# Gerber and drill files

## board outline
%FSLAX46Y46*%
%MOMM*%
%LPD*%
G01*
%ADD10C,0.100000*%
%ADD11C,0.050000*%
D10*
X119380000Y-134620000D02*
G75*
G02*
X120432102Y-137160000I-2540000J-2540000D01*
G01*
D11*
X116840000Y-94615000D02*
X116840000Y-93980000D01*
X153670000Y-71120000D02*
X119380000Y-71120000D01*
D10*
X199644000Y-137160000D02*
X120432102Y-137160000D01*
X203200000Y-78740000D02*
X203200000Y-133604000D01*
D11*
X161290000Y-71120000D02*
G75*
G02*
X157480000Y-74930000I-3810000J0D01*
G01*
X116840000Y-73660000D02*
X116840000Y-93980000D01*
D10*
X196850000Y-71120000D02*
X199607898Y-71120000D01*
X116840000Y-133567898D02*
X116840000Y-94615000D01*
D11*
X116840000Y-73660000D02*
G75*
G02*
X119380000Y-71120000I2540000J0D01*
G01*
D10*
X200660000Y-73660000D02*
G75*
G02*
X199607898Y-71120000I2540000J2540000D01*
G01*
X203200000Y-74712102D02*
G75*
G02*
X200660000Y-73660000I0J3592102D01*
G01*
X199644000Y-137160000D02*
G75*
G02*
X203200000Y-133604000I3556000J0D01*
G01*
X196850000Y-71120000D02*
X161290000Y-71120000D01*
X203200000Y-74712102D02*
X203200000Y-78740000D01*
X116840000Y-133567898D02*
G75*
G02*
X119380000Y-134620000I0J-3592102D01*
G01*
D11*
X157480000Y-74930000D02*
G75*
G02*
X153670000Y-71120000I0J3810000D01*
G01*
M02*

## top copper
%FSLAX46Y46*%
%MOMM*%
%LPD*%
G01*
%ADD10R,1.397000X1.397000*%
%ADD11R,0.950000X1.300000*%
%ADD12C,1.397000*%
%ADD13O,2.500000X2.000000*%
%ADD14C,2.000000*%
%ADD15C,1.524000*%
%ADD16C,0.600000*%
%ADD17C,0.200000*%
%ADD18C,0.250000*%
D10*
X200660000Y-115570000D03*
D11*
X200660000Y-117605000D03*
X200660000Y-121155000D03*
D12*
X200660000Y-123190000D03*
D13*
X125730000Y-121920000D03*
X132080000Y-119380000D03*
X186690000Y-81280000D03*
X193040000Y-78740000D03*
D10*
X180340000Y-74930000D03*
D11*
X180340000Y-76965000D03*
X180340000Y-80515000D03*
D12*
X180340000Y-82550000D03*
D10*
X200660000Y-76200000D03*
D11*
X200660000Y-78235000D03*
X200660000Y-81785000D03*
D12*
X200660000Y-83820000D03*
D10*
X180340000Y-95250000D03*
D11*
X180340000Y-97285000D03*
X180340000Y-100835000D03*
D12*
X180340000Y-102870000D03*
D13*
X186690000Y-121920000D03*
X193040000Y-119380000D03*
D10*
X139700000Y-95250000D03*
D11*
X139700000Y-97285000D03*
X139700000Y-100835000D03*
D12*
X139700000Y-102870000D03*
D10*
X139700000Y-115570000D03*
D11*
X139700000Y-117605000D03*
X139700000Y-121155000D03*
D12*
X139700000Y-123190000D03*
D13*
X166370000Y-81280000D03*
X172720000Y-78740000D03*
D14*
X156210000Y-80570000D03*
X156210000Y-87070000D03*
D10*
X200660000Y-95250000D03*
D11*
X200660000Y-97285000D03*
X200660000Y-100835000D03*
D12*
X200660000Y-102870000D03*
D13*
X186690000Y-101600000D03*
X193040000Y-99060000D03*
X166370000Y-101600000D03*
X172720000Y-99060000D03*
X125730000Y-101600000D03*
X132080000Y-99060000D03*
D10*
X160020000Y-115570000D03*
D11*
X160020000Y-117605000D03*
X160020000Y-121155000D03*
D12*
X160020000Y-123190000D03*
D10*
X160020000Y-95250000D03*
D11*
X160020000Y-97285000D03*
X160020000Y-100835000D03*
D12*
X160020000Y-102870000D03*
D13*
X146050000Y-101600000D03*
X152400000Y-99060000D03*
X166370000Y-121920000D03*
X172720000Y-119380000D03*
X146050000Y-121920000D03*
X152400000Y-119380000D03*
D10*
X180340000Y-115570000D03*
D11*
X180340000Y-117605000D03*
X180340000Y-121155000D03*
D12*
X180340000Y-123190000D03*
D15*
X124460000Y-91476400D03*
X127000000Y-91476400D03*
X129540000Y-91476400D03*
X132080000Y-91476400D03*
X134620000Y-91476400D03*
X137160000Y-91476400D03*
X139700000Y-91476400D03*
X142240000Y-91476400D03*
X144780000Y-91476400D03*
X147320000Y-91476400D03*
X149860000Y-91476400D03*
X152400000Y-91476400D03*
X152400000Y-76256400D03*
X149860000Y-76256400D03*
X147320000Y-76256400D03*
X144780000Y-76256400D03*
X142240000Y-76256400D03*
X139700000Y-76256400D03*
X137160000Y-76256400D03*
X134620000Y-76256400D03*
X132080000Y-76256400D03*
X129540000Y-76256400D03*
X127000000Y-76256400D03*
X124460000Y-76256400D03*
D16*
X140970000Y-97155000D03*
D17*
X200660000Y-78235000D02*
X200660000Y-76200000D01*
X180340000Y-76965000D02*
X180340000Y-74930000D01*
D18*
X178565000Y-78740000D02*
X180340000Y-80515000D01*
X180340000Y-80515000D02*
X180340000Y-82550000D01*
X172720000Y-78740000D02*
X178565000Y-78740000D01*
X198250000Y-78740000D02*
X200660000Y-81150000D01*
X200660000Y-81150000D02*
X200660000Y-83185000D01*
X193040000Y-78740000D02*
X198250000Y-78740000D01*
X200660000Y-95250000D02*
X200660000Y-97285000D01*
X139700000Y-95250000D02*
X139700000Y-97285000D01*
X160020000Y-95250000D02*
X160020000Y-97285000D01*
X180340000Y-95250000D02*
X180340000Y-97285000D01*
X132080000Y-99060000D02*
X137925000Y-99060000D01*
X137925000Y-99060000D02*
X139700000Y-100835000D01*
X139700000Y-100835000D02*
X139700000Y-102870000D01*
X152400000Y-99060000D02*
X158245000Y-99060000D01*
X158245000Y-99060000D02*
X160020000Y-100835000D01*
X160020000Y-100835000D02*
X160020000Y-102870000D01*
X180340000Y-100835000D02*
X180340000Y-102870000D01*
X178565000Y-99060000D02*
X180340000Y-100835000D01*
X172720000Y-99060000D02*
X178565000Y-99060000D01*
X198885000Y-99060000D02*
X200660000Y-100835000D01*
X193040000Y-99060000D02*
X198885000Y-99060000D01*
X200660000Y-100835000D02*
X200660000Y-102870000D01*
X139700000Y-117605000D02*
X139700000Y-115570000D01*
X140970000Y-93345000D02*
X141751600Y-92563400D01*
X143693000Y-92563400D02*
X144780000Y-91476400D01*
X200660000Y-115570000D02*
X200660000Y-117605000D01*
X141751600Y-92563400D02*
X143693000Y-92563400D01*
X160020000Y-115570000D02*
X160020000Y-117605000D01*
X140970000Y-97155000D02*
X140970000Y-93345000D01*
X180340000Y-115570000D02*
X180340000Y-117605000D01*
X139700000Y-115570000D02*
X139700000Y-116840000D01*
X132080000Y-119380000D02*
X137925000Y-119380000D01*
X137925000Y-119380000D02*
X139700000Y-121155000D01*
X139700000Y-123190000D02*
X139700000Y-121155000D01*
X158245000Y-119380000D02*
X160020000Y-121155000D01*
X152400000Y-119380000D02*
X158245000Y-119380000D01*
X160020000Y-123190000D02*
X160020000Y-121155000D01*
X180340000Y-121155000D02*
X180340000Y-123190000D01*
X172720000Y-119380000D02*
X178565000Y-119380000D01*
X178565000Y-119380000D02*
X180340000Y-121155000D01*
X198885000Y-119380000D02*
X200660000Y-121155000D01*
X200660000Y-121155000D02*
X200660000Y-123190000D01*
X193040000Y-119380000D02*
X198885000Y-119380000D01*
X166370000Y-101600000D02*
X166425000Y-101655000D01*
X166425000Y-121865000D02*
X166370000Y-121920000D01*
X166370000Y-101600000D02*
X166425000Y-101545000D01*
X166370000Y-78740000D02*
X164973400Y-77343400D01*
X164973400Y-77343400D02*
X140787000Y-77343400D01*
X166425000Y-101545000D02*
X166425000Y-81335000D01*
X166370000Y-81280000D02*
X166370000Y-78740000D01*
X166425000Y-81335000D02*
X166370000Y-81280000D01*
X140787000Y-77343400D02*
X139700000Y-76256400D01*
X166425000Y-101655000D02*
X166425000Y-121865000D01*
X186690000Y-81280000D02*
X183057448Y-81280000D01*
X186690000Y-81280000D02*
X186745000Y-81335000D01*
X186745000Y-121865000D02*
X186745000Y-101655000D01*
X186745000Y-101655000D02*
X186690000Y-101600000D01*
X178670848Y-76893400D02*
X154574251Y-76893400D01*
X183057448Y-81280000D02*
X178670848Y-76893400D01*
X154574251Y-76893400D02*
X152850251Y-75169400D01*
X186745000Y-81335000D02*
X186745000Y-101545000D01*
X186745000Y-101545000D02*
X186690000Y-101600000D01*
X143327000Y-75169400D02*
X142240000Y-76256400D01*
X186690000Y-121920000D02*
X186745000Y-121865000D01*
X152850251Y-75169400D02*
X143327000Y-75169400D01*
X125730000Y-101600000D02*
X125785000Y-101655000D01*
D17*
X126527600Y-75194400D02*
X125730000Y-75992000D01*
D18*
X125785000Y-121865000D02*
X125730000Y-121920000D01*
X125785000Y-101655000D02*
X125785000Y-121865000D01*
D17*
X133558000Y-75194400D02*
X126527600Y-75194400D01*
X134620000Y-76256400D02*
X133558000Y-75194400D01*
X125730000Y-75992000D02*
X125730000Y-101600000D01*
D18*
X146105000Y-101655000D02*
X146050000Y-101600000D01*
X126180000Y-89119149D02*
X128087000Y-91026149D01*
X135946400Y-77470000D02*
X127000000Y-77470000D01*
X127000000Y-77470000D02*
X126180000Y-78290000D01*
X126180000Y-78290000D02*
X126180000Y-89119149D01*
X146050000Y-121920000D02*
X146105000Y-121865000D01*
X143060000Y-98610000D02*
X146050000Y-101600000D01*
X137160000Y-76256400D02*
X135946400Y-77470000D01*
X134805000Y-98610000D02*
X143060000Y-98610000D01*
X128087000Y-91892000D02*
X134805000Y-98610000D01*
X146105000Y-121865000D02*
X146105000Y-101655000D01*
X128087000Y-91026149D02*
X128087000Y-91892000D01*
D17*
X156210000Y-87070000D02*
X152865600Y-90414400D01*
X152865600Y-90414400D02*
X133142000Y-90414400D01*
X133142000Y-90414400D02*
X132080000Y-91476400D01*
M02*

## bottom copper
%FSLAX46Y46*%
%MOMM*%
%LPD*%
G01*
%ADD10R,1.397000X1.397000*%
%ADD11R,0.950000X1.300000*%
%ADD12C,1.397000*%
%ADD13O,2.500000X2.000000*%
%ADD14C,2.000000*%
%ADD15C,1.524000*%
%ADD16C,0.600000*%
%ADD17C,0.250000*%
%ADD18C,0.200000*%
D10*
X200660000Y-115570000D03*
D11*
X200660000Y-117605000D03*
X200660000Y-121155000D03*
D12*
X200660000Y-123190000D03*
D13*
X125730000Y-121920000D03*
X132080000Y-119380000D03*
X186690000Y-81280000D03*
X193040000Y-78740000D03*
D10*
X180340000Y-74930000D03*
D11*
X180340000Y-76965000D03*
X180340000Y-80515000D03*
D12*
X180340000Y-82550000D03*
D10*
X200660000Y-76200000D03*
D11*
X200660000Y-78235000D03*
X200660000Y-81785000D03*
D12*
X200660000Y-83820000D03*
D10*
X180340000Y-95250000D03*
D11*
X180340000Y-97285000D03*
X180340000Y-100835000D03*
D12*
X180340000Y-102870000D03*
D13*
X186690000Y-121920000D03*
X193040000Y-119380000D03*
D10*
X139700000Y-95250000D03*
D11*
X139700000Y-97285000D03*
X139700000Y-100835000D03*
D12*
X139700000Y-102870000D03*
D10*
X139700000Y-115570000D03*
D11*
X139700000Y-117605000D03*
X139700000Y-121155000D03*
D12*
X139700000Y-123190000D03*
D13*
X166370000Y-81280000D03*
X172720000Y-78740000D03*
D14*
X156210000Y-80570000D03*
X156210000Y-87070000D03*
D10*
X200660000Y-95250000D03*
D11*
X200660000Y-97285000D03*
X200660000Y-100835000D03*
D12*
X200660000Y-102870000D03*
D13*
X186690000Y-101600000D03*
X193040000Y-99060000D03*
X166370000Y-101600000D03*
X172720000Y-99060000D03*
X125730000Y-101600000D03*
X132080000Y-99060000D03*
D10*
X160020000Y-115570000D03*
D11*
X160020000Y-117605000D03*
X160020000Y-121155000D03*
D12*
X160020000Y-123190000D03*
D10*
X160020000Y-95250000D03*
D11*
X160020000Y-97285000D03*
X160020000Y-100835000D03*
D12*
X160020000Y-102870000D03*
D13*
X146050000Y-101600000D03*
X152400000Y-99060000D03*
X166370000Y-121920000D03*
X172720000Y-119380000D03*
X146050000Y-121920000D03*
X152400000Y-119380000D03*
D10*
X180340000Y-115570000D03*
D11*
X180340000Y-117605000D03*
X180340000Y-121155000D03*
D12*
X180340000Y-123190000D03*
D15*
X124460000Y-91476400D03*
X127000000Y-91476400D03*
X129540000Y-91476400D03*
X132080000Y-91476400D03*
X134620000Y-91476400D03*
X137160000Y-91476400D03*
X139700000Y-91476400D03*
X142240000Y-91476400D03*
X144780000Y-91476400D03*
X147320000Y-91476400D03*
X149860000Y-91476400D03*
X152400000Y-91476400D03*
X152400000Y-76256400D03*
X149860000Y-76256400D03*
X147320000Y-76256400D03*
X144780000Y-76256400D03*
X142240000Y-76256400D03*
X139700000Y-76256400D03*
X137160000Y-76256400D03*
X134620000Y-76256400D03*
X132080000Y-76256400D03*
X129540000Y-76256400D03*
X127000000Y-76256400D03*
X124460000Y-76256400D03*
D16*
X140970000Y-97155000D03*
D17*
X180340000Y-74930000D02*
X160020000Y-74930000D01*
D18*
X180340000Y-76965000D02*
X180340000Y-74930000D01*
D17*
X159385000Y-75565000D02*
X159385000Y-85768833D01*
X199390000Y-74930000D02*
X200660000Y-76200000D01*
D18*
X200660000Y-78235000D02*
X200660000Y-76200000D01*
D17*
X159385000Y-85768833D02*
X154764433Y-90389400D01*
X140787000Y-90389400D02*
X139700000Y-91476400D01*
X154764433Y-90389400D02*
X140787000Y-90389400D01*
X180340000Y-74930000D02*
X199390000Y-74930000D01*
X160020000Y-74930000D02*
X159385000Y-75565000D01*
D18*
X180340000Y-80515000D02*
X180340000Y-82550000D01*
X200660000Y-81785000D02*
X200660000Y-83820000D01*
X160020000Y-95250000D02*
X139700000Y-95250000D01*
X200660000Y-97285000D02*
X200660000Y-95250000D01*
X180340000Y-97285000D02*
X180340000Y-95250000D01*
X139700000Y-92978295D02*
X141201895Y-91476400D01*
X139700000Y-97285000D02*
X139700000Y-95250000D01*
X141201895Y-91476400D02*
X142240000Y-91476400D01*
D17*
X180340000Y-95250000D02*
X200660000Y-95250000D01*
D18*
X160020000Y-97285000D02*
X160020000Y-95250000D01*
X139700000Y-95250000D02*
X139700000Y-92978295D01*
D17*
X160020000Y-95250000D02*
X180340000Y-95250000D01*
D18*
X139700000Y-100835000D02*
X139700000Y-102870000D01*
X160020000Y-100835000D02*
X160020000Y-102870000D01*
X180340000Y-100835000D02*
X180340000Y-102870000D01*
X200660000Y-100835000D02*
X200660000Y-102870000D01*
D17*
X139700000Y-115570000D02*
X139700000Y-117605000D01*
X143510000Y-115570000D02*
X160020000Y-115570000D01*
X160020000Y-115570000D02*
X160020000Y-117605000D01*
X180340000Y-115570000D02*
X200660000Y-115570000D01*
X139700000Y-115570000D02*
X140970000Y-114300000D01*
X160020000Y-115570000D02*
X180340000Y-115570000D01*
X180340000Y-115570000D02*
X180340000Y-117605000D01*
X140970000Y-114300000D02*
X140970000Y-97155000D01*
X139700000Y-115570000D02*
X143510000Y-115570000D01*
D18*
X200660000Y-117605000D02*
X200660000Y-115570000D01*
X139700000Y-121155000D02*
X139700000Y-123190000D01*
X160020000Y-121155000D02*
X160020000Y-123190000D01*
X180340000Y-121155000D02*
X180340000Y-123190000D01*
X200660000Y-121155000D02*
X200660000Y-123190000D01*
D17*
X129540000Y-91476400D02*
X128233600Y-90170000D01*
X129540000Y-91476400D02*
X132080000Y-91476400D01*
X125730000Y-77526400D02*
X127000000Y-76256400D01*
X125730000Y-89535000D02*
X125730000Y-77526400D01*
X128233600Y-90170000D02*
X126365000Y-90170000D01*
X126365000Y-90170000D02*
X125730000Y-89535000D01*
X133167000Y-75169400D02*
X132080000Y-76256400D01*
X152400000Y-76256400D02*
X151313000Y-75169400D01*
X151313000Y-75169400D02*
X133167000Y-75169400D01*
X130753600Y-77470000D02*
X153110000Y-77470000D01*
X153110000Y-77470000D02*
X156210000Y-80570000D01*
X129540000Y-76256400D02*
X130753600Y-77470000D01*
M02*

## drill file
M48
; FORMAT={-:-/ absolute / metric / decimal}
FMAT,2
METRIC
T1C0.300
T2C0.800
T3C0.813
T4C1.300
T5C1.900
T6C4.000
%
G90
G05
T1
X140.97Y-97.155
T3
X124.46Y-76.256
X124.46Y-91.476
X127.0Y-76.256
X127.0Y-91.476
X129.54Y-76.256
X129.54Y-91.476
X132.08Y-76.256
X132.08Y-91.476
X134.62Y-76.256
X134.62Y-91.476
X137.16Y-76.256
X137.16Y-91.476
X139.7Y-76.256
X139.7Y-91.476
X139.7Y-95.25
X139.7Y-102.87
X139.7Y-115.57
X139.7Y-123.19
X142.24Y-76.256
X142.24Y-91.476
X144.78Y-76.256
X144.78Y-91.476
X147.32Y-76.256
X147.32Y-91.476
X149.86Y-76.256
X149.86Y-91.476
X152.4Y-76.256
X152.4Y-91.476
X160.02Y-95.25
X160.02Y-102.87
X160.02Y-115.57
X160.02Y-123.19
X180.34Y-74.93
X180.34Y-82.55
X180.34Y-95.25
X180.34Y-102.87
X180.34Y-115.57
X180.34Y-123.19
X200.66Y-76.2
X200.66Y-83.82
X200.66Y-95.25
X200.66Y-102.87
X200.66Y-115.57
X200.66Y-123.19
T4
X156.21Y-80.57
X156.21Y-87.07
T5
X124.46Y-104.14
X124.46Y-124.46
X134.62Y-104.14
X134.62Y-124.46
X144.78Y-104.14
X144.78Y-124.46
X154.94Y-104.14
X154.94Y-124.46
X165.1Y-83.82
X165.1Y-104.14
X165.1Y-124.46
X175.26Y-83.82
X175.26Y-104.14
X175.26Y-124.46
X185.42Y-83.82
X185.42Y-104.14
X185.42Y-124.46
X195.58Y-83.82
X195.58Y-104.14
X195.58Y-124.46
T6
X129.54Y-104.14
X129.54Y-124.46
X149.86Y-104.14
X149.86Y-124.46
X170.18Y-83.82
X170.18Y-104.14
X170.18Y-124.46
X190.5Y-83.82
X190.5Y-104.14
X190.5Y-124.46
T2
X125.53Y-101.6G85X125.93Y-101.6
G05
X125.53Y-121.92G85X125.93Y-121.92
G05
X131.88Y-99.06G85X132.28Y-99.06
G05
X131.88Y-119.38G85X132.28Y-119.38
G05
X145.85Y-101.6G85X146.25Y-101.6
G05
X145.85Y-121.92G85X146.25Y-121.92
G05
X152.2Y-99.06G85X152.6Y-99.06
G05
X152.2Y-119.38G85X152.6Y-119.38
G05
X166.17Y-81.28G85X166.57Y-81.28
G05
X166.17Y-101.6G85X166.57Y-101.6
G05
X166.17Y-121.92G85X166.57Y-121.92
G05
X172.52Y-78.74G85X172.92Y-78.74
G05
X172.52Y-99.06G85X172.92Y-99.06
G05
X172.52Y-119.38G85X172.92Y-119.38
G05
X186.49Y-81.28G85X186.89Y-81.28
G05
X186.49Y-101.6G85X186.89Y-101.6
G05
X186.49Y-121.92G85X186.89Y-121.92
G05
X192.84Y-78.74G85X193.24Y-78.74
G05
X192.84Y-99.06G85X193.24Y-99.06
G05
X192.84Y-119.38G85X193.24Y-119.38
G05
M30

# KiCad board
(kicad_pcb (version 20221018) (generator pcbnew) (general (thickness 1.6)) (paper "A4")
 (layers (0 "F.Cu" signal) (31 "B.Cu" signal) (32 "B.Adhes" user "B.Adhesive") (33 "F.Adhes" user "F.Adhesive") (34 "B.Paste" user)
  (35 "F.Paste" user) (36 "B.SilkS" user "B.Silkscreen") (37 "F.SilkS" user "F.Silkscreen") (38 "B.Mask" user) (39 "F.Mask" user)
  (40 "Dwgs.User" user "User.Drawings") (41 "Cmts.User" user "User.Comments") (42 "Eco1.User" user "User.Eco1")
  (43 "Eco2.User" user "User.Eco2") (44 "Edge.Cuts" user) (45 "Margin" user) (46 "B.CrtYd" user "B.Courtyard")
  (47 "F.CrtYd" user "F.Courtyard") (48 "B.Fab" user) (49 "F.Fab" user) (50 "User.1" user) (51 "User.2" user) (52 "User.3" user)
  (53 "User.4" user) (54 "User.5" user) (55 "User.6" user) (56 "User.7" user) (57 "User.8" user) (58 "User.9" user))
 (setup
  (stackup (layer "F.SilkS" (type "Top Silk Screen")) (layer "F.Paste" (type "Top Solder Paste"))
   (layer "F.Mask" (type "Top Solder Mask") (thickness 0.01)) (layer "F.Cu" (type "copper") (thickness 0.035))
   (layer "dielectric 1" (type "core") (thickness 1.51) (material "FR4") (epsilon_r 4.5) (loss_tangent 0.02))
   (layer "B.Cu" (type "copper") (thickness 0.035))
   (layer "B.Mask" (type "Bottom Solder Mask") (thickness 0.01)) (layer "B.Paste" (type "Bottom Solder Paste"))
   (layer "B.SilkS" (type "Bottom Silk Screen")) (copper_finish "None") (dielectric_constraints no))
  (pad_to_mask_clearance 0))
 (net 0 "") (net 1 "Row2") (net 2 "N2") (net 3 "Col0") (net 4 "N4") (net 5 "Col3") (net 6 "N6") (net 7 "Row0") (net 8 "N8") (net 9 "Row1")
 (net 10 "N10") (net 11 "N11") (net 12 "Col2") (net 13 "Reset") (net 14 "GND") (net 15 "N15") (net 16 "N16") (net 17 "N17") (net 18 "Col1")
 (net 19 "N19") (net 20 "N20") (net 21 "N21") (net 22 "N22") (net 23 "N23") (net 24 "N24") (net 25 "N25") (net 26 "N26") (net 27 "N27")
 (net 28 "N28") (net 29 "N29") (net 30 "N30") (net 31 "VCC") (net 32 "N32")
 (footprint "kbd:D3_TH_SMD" (layer "F.Cu") (at 200.66 119.38 -90)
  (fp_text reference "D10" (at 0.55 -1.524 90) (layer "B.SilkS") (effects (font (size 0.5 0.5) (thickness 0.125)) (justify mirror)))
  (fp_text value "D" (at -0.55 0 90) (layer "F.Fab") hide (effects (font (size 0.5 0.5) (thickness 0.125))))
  (pad "1" thru_hole rect (at -3.81 0 270) (size 1.397 1.397) (drill 0.8128) (layers "*.Cu" "*.Mask" "F.SilkS") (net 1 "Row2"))
  (pad "1" smd rect (at -1.775 0 270) (size 1.3 0.95) (layers "F.Cu" "F.Paste" "F.Mask") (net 1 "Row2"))
  (pad "1" smd rect (at -1.775 0 270) (size 1.3 0.95) (layers "B.Cu" "B.Paste" "B.Mask") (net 1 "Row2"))
  (pad "2" smd rect (at 1.775 0 270) (size 1.3 0.95) (layers "F.Cu" "F.Paste" "F.Mask") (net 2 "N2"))
  (pad "2" smd rect (at 1.775 0 270) (size 1.3 0.95) (layers "B.Cu" "B.Paste" "B.Mask") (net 2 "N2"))
  (pad "2" thru_hole circle (at 3.81 0 270) (size 1.397 1.397) (drill 0.8128) (layers "*.Cu" "*.Mask" "F.SilkS") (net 2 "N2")))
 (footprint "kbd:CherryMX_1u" (layer "F.Cu") (at 129.54 124.46)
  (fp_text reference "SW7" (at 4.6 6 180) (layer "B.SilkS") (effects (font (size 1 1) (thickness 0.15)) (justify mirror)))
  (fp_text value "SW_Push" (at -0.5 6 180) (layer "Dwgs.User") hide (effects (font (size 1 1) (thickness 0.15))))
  (pad "" np_thru_hole circle (at -5.08 0 90) (size 1.9 1.9) (drill 1.9) (layers "*.Cu" "*.Mask"))
  (pad "" np_thru_hole circle (at 0 0 90) (size 4 4) (drill 4) (layers "*.Cu" "*.Mask"))
  (pad "" np_thru_hole circle (at 5.08 0 90) (size 1.9 1.9) (drill 1.9) (layers "*.Cu" "*.Mask"))
  (pad "1" thru_hole oval (at -3.81 -2.54) (size 2.5 2) (drill oval 1.2 0.8) (layers "*.Cu" "F.SilkS" "B.Mask") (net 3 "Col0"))
  (pad "2" thru_hole oval (at 2.54 -5.08) (size 2.5 2) (drill oval 1.2 0.8) (layers "*.Cu" "F.SilkS" "B.Mask") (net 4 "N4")))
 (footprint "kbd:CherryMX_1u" (layer "F.Cu") (at 190.5 83.82)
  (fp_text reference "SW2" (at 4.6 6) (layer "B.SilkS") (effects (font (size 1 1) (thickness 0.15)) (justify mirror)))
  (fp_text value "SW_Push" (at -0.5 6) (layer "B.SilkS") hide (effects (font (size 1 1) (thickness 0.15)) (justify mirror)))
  (pad "" np_thru_hole circle (at -5.08 0 90) (size 1.9 1.9) (drill 1.9) (layers "*.Cu" "*.Mask"))
  (pad "" np_thru_hole circle (at 0 0 90) (size 4 4) (drill 4) (layers "*.Cu" "*.Mask"))
  (pad "" np_thru_hole circle (at 5.08 0 90) (size 1.9 1.9) (drill 1.9) (layers "*.Cu" "*.Mask"))
  (pad "1" thru_hole oval (at -3.81 -2.54) (size 2.5 2) (drill oval 1.2 0.8) (layers "*.Cu" "F.SilkS" "B.Mask") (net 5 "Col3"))
  (pad "2" thru_hole oval (at 2.54 -5.08) (size 2.5 2) (drill oval 1.2 0.8) (layers "*.Cu" "F.SilkS" "B.Mask") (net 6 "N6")))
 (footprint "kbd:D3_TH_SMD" (layer "F.Cu") (at 180.34 78.74 -90)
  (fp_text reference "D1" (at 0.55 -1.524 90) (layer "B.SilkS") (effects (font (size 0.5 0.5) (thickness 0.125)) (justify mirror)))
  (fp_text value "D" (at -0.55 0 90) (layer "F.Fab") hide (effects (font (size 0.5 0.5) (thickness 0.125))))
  (pad "1" thru_hole rect (at -3.81 0 270) (size 1.397 1.397) (drill 0.8128) (layers "*.Cu" "*.Mask" "F.SilkS") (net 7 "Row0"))
  (pad "1" smd rect (at -1.775 0 270) (size 1.3 0.95) (layers "F.Cu" "F.Paste" "F.Mask") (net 7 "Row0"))
  (pad "1" smd rect (at -1.775 0 270) (size 1.3 0.95) (layers "B.Cu" "B.Paste" "B.Mask") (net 7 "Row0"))
  (pad "2" smd rect (at 1.775 0 270) (size 1.3 0.95) (layers "F.Cu" "F.Paste" "F.Mask") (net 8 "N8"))
  (pad "2" smd rect (at 1.775 0 270) (size 1.3 0.95) (layers "B.Cu" "B.Paste" "B.Mask") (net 8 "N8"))
  (pad "2" thru_hole circle (at 3.81 0 270) (size 1.397 1.397) (drill 0.8128) (layers "*.Cu" "*.Mask" "F.SilkS") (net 8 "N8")))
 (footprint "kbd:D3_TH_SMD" (layer "F.Cu") (at 200.66 80.01 -90)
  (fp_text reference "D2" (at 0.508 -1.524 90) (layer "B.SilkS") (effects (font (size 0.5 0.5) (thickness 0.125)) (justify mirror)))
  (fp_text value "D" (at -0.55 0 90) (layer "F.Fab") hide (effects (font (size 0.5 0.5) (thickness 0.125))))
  (pad "1" thru_hole rect (at -3.81 0 270) (size 1.397 1.397) (drill 0.8128) (layers "*.Cu" "*.Mask" "F.SilkS") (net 7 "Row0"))
  (pad "1" smd rect (at -1.775 0 270) (size 1.3 0.95) (layers "F.Cu" "F.Paste" "F.Mask") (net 7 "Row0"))
  (pad "1" smd rect (at -1.775 0 270) (size 1.3 0.95) (layers "B.Cu" "B.Paste" "B.Mask") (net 7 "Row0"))
  (pad "2" smd rect (at 1.775 0 270) (size 1.3 0.95) (layers "F.Cu" "F.Paste" "F.Mask") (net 6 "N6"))
  (pad "2" smd rect (at 1.775 0 270) (size 1.3 0.95) (layers "B.Cu" "B.Paste" "B.Mask") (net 6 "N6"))
  (pad "2" thru_hole circle (at 3.81 0 270) (size 1.397 1.397) (drill 0.8128) (layers "*.Cu" "*.Mask" "F.SilkS") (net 6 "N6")))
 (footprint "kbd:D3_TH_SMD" (layer "F.Cu") (at 180.34 99.06 -90)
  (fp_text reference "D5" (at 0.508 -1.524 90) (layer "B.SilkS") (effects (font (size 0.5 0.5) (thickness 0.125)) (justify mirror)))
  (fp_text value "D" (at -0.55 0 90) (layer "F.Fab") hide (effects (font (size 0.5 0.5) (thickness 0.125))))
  (pad "1" thru_hole rect (at -3.81 0 270) (size 1.397 1.397) (drill 0.8128) (layers "*.Cu" "*.Mask" "F.SilkS") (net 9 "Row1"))
  (pad "1" smd rect (at -1.775 0 270) (size 1.3 0.95) (layers "F.Cu" "F.Paste" "F.Mask") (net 9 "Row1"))
  (pad "1" smd rect (at -1.775 0 270) (size 1.3 0.95) (layers "B.Cu" "B.Paste" "B.Mask") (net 9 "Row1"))
  (pad "2" smd rect (at 1.775 0 270) (size 1.3 0.95) (layers "F.Cu" "F.Paste" "F.Mask") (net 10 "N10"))
  (pad "2" smd rect (at 1.775 0 270) (size 1.3 0.95) (layers "B.Cu" "B.Paste" "B.Mask") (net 10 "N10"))
  (pad "2" thru_hole circle (at 3.81 0 270) (size 1.397 1.397) (drill 0.8128) (layers "*.Cu" "*.Mask" "F.SilkS") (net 10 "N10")))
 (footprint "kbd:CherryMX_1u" (layer "F.Cu") (at 190.5 124.46)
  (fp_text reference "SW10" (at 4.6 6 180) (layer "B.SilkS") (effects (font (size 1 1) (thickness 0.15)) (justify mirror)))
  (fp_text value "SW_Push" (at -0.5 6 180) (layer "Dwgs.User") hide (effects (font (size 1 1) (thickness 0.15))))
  (pad "" np_thru_hole circle (at -5.08 0 90) (size 1.9 1.9) (drill 1.9) (layers "*.Cu" "*.Mask"))
  (pad "" np_thru_hole circle (at 0 0 90) (size 4 4) (drill 4) (layers "*.Cu" "*.Mask"))
  (pad "" np_thru_hole circle (at 5.08 0 90) (size 1.9 1.9) (drill 1.9) (layers "*.Cu" "*.Mask"))
  (pad "1" thru_hole oval (at -3.81 -2.54) (size 2.5 2) (drill oval 1.2 0.8) (layers "*.Cu" "F.SilkS" "B.Mask") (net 5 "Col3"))
  (pad "2" thru_hole oval (at 2.54 -5.08) (size 2.5 2) (drill oval 1.2 0.8) (layers "*.Cu" "F.SilkS" "B.Mask") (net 2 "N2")))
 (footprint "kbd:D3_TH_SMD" (layer "F.Cu") (at 139.7 99.06 -90)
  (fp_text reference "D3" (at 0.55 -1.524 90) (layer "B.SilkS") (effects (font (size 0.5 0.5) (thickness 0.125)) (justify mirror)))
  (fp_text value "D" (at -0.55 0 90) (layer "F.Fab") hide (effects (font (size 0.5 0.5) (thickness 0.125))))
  (pad "1" thru_hole rect (at -3.81 0 270) (size 1.397 1.397) (drill 0.8128) (layers "*.Cu" "*.Mask" "F.SilkS") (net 9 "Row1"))
  (pad "1" smd rect (at -1.775 0 270) (size 1.3 0.95) (layers "F.Cu" "F.Paste" "F.Mask") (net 9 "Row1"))
  (pad "1" smd rect (at -1.775 0 270) (size 1.3 0.95) (layers "B.Cu" "B.Paste" "B.Mask") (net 9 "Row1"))
  (pad "2" smd rect (at 1.775 0 270) (size 1.3 0.95) (layers "F.Cu" "F.Paste" "F.Mask") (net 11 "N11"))
  (pad "2" smd rect (at 1.775 0 270) (size 1.3 0.95) (layers "B.Cu" "B.Paste" "B.Mask") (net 11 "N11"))
  (pad "2" thru_hole circle (at 3.81 0 270) (size 1.397 1.397) (drill 0.8128) (layers "*.Cu" "*.Mask" "F.SilkS") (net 11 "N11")))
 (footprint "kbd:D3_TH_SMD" (layer "F.Cu") (at 139.7 119.38 -90)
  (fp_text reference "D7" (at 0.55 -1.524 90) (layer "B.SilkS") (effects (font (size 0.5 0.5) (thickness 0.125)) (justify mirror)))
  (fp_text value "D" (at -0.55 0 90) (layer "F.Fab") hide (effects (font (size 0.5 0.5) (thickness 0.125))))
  (pad "1" thru_hole rect (at -3.81 0 270) (size 1.397 1.397) (drill 0.8128) (layers "*.Cu" "*.Mask" "F.SilkS") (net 1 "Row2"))
  (pad "1" smd rect (at -1.775 0 270) (size 1.3 0.95) (layers "F.Cu" "F.Paste" "F.Mask") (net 1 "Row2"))
  (pad "1" smd rect (at -1.775 0 270) (size 1.3 0.95) (layers "B.Cu" "B.Paste" "B.Mask") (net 1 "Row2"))
  (pad "2" smd rect (at 1.775 0 270) (size 1.3 0.95) (layers "F.Cu" "F.Paste" "F.Mask") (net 4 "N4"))
  (pad "2" smd rect (at 1.775 0 270) (size 1.3 0.95) (layers "B.Cu" "B.Paste" "B.Mask") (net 4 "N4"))
  (pad "2" thru_hole circle (at 3.81 0 270) (size 1.397 1.397) (drill 0.8128) (layers "*.Cu" "*.Mask" "F.SilkS") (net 4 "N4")))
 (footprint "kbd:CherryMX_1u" (layer "F.Cu") (at 170.18 83.82)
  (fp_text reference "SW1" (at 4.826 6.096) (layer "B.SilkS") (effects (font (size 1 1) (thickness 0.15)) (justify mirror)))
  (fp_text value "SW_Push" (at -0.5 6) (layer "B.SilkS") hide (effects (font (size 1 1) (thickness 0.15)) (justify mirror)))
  (pad "" np_thru_hole circle (at -5.08 0 90) (size 1.9 1.9) (drill 1.9) (layers "*.Cu" "*.Mask"))
  (pad "" np_thru_hole circle (at 0 0 90) (size 4 4) (drill 4) (layers "*.Cu" "*.Mask"))
  (pad "" np_thru_hole circle (at 5.08 0 90) (size 1.9 1.9) (drill 1.9) (layers "*.Cu" "*.Mask"))
  (pad "1" thru_hole oval (at -3.81 -2.54) (size 2.5 2) (drill oval 1.2 0.8) (layers "*.Cu" "F.SilkS" "B.Mask") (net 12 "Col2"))
  (pad "2" thru_hole oval (at 2.54 -5.08) (size 2.5 2) (drill oval 1.2 0.8) (layers "*.Cu" "F.SilkS" "B.Mask") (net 8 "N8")))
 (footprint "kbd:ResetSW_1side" (layer "F.Cu") (at 156.21 83.82 90)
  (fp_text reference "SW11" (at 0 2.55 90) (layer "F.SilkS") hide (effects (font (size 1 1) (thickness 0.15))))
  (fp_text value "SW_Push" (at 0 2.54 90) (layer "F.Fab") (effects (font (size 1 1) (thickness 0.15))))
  (pad "1" thru_hole circle (at 3.25 0 90) (size 2 2) (drill 1.3) (layers "*.Cu" "B.Mask") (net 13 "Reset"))
  (pad "2" thru_hole circle (at -3.25 0 90) (size 2 2) (drill 1.3) (layers "*.Cu" "B.Mask") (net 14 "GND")))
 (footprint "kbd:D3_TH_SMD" (layer "F.Cu") (at 200.66 99.06 -90)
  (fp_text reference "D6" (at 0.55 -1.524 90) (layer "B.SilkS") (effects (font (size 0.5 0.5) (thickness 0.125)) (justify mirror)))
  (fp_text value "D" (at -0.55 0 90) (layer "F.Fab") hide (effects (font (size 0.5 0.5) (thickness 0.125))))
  (pad "1" thru_hole rect (at -3.81 0 270) (size 1.397 1.397) (drill 0.8128) (layers "*.Cu" "*.Mask" "F.SilkS") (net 9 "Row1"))
  (pad "1" smd rect (at -1.775 0 270) (size 1.3 0.95) (layers "F.Cu" "F.Paste" "F.Mask") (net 9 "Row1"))
  (pad "1" smd rect (at -1.775 0 270) (size 1.3 0.95) (layers "B.Cu" "B.Paste" "B.Mask") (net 9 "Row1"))
  (pad "2" smd rect (at 1.775 0 270) (size 1.3 0.95) (layers "F.Cu" "F.Paste" "F.Mask") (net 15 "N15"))
  (pad "2" smd rect (at 1.775 0 270) (size 1.3 0.95) (layers "B.Cu" "B.Paste" "B.Mask") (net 15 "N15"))
  (pad "2" thru_hole circle (at 3.81 0 270) (size 1.397 1.397) (drill 0.8128) (layers "*.Cu" "*.Mask" "F.SilkS") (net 15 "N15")))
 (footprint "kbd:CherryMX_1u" (layer "F.Cu") (at 190.5 104.14)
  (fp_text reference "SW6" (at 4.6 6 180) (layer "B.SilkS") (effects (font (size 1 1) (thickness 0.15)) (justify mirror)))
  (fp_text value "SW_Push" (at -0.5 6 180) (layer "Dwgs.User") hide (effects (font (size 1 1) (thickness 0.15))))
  (pad "" np_thru_hole circle (at -5.08 0 90) (size 1.9 1.9) (drill 1.9) (layers "*.Cu" "*.Mask"))
  (pad "" np_thru_hole circle (at 0 0 90) (size 4 4) (drill 4) (layers "*.Cu" "*.Mask"))
  (pad "" np_thru_hole circle (at 5.08 0 90) (size 1.9 1.9) (drill 1.9) (layers "*.Cu" "*.Mask"))
  (pad "1" thru_hole oval (at -3.81 -2.54) (size 2.5 2) (drill oval 1.2 0.8) (layers "*.Cu" "F.SilkS" "B.Mask") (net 5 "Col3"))
  (pad "2" thru_hole oval (at 2.54 -5.08) (size 2.5 2) (drill oval 1.2 0.8) (layers "*.Cu" "F.SilkS" "B.Mask") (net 15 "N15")))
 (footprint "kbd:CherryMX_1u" (layer "F.Cu") (at 170.18 104.14)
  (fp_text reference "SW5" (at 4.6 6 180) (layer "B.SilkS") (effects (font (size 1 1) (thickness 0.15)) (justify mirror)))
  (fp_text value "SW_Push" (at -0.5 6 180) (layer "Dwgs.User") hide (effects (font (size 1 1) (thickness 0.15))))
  (pad "" np_thru_hole circle (at -5.08 0 90) (size 1.9 1.9) (drill 1.9) (layers "*.Cu" "*.Mask"))
  (pad "" np_thru_hole circle (at 0 0 90) (size 4 4) (drill 4) (layers "*.Cu" "*.Mask"))
  (pad "" np_thru_hole circle (at 5.08 0 90) (size 1.9 1.9) (drill 1.9) (layers "*.Cu" "*.Mask"))
  (pad "1" thru_hole oval (at -3.81 -2.54) (size 2.5 2) (drill oval 1.2 0.8) (layers "*.Cu" "F.SilkS" "B.Mask") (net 12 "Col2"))
  (pad "2" thru_hole oval (at 2.54 -5.08) (size 2.5 2) (drill oval 1.2 0.8) (layers "*.Cu" "F.SilkS" "B.Mask") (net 10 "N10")))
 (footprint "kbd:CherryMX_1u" (layer "F.Cu") (at 129.54 104.14)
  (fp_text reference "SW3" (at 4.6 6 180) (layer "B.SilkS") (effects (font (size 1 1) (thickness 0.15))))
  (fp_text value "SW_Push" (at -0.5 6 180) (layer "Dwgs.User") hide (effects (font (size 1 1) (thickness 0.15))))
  (pad "" np_thru_hole circle (at -5.08 0 90) (size 1.9 1.9) (drill 1.9) (layers "*.Cu" "*.Mask"))
  (pad "" np_thru_hole circle (at 0 0 90) (size 4 4) (drill 4) (layers "*.Cu" "*.Mask"))
  (pad "" np_thru_hole circle (at 5.08 0 90) (size 1.9 1.9) (drill 1.9) (layers "*.Cu" "*.Mask"))
  (pad "1" thru_hole oval (at -3.81 -2.54) (size 2.5 2) (drill oval 1.2 0.8) (layers "*.Cu" "F.SilkS" "B.Mask") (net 3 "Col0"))
  (pad "2" thru_hole oval (at 2.54 -5.08) (size 2.5 2) (drill oval 1.2 0.8) (layers "*.Cu" "F.SilkS" "B.Mask") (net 11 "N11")))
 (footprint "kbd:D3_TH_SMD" (layer "F.Cu") (at 160.02 119.38 -90)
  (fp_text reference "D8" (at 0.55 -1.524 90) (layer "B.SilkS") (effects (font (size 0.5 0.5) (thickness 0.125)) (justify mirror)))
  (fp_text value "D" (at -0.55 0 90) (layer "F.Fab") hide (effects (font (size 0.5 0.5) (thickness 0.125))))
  (pad "1" thru_hole rect (at -3.81 0 270) (size 1.397 1.397) (drill 0.8128) (layers "*.Cu" "*.Mask" "F.SilkS") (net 1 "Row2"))
  (pad "1" smd rect (at -1.775 0 270) (size 1.3 0.95) (layers "F.Cu" "F.Paste" "F.Mask") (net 1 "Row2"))
  (pad "1" smd rect (at -1.775 0 270) (size 1.3 0.95) (layers "B.Cu" "B.Paste" "B.Mask") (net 1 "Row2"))
  (pad "2" smd rect (at 1.775 0 270) (size 1.3 0.95) (layers "F.Cu" "F.Paste" "F.Mask") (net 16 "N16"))
  (pad "2" smd rect (at 1.775 0 270) (size 1.3 0.95) (layers "B.Cu" "B.Paste" "B.Mask") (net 16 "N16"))
  (pad "2" thru_hole circle (at 3.81 0 270) (size 1.397 1.397) (drill 0.8128) (layers "*.Cu" "*.Mask" "F.SilkS") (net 16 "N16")))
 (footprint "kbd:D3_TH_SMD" (layer "F.Cu") (at 160.02 99.06 -90)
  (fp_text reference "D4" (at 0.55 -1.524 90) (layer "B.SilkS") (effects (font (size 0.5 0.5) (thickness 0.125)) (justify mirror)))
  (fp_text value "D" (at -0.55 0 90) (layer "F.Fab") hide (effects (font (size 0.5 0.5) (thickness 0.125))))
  (pad "1" thru_hole rect (at -3.81 0 270) (size 1.397 1.397) (drill 0.8128) (layers "*.Cu" "*.Mask" "F.SilkS") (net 9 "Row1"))
  (pad "1" smd rect (at -1.775 0 270) (size 1.3 0.95) (layers "F.Cu" "F.Paste" "F.Mask") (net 9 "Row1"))
  (pad "1" smd rect (at -1.775 0 270) (size 1.3 0.95) (layers "B.Cu" "B.Paste" "B.Mask") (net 9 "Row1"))
  (pad "2" smd rect (at 1.775 0 270) (size 1.3 0.95) (layers "F.Cu" "F.Paste" "F.Mask") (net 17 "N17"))
  (pad "2" smd rect (at 1.775 0 270) (size 1.3 0.95) (layers "B.Cu" "B.Paste" "B.Mask") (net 17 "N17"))
  (pad "2" thru_hole circle (at 3.81 0 270) (size 1.397 1.397) (drill 0.8128) (layers "*.Cu" "*.Mask" "F.SilkS") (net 17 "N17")))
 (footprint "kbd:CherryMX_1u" (layer "F.Cu") (at 149.86 104.14)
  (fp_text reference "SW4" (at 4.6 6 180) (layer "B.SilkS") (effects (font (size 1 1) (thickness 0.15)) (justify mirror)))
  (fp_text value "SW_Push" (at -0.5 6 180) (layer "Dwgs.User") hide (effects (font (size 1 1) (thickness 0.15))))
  (pad "" np_thru_hole circle (at -5.08 0 90) (size 1.9 1.9) (drill 1.9) (layers "*.Cu" "*.Mask"))
  (pad "" np_thru_hole circle (at 0 0 90) (size 4 4) (drill 4) (layers "*.Cu" "*.Mask"))
  (pad "" np_thru_hole circle (at 5.08 0 90) (size 1.9 1.9) (drill 1.9) (layers "*.Cu" "*.Mask"))
  (pad "1" thru_hole oval (at -3.81 -2.54) (size 2.5 2) (drill oval 1.2 0.8) (layers "*.Cu" "F.SilkS" "B.Mask") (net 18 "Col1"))
  (pad "2" thru_hole oval (at 2.54 -5.08) (size 2.5 2) (drill oval 1.2 0.8) (layers "*.Cu" "F.SilkS" "B.Mask") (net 17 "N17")))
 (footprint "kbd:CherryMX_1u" (layer "F.Cu") (at 170.18 124.46)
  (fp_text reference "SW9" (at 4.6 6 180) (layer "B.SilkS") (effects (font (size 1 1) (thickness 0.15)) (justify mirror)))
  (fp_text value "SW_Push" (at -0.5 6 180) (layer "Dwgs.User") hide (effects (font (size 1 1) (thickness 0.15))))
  (pad "" np_thru_hole circle (at -5.08 0 90) (size 1.9 1.9) (drill 1.9) (layers "*.Cu" "*.Mask"))
  (pad "" np_thru_hole circle (at 0 0 90) (size 4 4) (drill 4) (layers "*.Cu" "*.Mask"))
  (pad "" np_thru_hole circle (at 5.08 0 90) (size 1.9 1.9) (drill 1.9) (layers "*.Cu" "*.Mask"))
  (pad "1" thru_hole oval (at -3.81 -2.54) (size 2.5 2) (drill oval 1.2 0.8) (layers "*.Cu" "F.SilkS" "B.Mask") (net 12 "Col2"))
  (pad "2" thru_hole oval (at 2.54 -5.08) (size 2.5 2) (drill oval 1.2 0.8) (layers "*.Cu" "F.SilkS" "B.Mask") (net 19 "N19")))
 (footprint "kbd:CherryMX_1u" (layer "F.Cu") (at 149.86 124.46)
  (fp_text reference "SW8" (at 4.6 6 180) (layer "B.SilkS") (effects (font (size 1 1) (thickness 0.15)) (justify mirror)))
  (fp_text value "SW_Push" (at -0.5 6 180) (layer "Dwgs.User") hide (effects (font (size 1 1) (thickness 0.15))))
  (pad "" np_thru_hole circle (at -5.08 0 90) (size 1.9 1.9) (drill 1.9) (layers "*.Cu" "*.Mask"))
  (pad "" np_thru_hole circle (at 0 0 90) (size 4 4) (drill 4) (layers "*.Cu" "*.Mask"))
  (pad "" np_thru_hole circle (at 5.08 0 90) (size 1.9 1.9) (drill 1.9) (layers "*.Cu" "*.Mask"))
  (pad "1" thru_hole oval (at -3.81 -2.54) (size 2.5 2) (drill oval 1.2 0.8) (layers "*.Cu" "F.SilkS" "B.Mask") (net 18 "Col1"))
  (pad "2" thru_hole oval (at 2.54 -5.08) (size 2.5 2) (drill oval 1.2 0.8) (layers "*.Cu" "F.SilkS" "B.Mask") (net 16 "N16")))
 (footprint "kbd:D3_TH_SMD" (layer "F.Cu") (at 180.34 119.38 -90)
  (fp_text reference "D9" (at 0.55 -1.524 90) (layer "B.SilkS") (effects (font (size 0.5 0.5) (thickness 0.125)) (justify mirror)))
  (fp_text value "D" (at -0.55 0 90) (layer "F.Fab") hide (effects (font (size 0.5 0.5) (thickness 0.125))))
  (pad "1" thru_hole rect (at -3.81 0 270) (size 1.397 1.397) (drill 0.8128) (layers "*.Cu" "*.Mask" "F.SilkS") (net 1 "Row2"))
  (pad "1" smd rect (at -1.775 0 270) (size 1.3 0.95) (layers "F.Cu" "F.Paste" "F.Mask") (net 1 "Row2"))
  (pad "1" smd rect (at -1.775 0 270) (size 1.3 0.95) (layers "B.Cu" "B.Paste" "B.Mask") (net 1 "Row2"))
  (pad "2" smd rect (at 1.775 0 270) (size 1.3 0.95) (layers "F.Cu" "F.Paste" "F.Mask") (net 19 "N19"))
  (pad "2" smd rect (at 1.775 0 270) (size 1.3 0.95) (layers "B.Cu" "B.Paste" "B.Mask") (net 19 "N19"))
  (pad "2" thru_hole circle (at 3.81 0 270) (size 1.397 1.397) (drill 0.8128) (layers "*.Cu" "*.Mask" "F.SilkS") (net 19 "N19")))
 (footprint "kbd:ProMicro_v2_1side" (layer "B.Cu") (at 138.938 83.82 -90)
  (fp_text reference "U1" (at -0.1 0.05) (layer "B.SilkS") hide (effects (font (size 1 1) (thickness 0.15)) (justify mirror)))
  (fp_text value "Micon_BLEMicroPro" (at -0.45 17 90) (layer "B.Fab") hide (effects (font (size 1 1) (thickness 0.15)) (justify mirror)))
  (pad "1" thru_hole circle (at 7.6564 14.478 270) (size 1.524 1.524) (drill 0.8128) (layers "*.Cu" "B.SilkS" "B.Mask") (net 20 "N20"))
  (pad "2" thru_hole circle (at 7.6564 11.938 270) (size 1.524 1.524) (drill 0.8128) (layers "*.Cu" "B.SilkS" "B.Mask") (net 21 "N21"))
  (pad "3" thru_hole circle (at 7.6564 9.398 270) (size 1.524 1.524) (drill 0.8128) (layers "*.Cu" "B.SilkS" "B.Mask") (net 14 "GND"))
  (pad "4" thru_hole circle (at 7.6564 6.858 270) (size 1.524 1.524) (drill 0.8128) (layers "*.Cu" "B.SilkS" "B.Mask") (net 14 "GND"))
  (pad "5" thru_hole circle (at 7.6564 4.318 270) (size 1.524 1.524) (drill 0.8128) (layers "*.Cu" "B.SilkS" "B.Mask") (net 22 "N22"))
  (pad "6" thru_hole circle (at 7.6564 1.778 270) (size 1.524 1.524) (drill 0.8128) (layers "*.Cu" "B.SilkS" "B.Mask") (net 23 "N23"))
  (pad "7" thru_hole circle (at 7.6564 -0.762 270) (size 1.524 1.524) (drill 0.8128) (layers "*.Cu" "B.SilkS" "B.Mask") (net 7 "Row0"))
  (pad "8" thru_hole circle (at 7.6564 -3.302 270) (size 1.524 1.524) (drill 0.8128) (layers "*.Cu" "B.SilkS" "B.Mask") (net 9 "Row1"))
  (pad "9" thru_hole circle (at 7.6564 -5.842 270) (size 1.524 1.524) (drill 0.8128) (layers "*.Cu" "B.SilkS" "B.Mask") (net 1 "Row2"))
  (pad "10" thru_hole circle (at 7.6564 -8.382 270) (size 1.524 1.524) (drill 0.8128) (layers "*.Cu" "B.SilkS" "B.Mask") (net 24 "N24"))
  (pad "11" thru_hole circle (at 7.6564 -10.922 270) (size 1.524 1.524) (drill 0.8128) (layers "*.Cu" "B.SilkS" "B.Mask") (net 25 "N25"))
  (pad "12" thru_hole circle (at 7.6564 -13.462 270) (size 1.524 1.524) (drill 0.8128) (layers "*.Cu" "B.SilkS" "B.Mask") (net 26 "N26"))
  (pad "13" thru_hole circle (at -7.5636 -13.462 270) (size 1.524 1.524) (drill 0.8128) (layers "*.Cu" "B.SilkS" "B.Mask") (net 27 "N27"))
  (pad "14" thru_hole circle (at -7.5636 -10.922 270) (size 1.524 1.524) (drill 0.8128) (layers "*.Cu" "B.SilkS" "B.Mask") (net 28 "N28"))
  (pad "15" thru_hole circle (at -7.5636 -8.382 270) (size 1.524 1.524) (drill 0.8128) (layers "*.Cu" "B.SilkS" "B.Mask") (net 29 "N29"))
  (pad "16" thru_hole circle (at -7.5636 -5.842 270) (size 1.524 1.524) (drill 0.8128) (layers "*.Cu" "B.SilkS" "B.Mask") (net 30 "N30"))
  (pad "17" thru_hole circle (at -7.5636 -3.302 270) (size 1.524 1.524) (drill 0.8128) (layers "*.Cu" "B.SilkS" "B.Mask") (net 5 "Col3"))
  (pad "18" thru_hole circle (at -7.5636 -0.762 270) (size 1.524 1.524) (drill 0.8128) (layers "*.Cu" "B.SilkS" "B.Mask") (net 12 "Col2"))
  (pad "19" thru_hole circle (at -7.5636 1.778 270) (size 1.524 1.524) (drill 0.8128) (layers "*.Cu" "B.SilkS" "B.Mask") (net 18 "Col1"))
  (pad "20" thru_hole circle (at -7.5636 4.318 270) (size 1.524 1.524) (drill 0.8128) (layers "*.Cu" "B.SilkS" "B.Mask") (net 3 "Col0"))
  (pad "21" thru_hole circle (at -7.5636 6.858 270) (size 1.524 1.524) (drill 0.8128) (layers "*.Cu" "B.SilkS" "B.Mask") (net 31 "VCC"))
  (pad "22" thru_hole circle (at -7.5636 9.398 270) (size 1.524 1.524) (drill 0.8128) (layers "*.Cu" "B.SilkS" "B.Mask") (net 13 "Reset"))
  (pad "23" thru_hole circle (at -7.5636 11.938 270) (size 1.524 1.524) (drill 0.8128) (layers "*.Cu" "B.SilkS" "B.Mask") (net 14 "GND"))
  (pad "24" thru_hole circle (at -7.5636 14.478 270) (size 1.524 1.524) (drill 0.8128) (layers "*.Cu" "B.SilkS" "B.Mask") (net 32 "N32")))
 (gr_arc (start 119.38 134.62) (mid 120.15867 135.785362) (end 120.432102 137.16) (stroke (width 0.1) (type default)) (layer "Edge.Cuts"))
 (gr_line (start 116.84 94.615) (end 116.84 93.98) (stroke (width 0.05) (type default)) (layer "Edge.Cuts"))
 (gr_line (start 153.67 71.12) (end 119.38 71.12) (stroke (width 0.05) (type default)) (layer "Edge.Cuts"))
 (gr_line (start 199.644 137.16) (end 120.432102 137.16) (stroke (width 0.1) (type default)) (layer "Edge.Cuts"))
 (gr_line (start 203.2 78.74) (end 203.2 133.604) (stroke (width 0.1) (type default)) (layer "Edge.Cuts"))
 (gr_arc (start 161.29 71.12) (mid 160.174077 73.814077) (end 157.48 74.93) (stroke (width 0.05) (type default)) (layer "Edge.Cuts"))
 (gr_line (start 116.84 73.66) (end 116.84 93.98) (stroke (width 0.05) (type default)) (layer "Edge.Cuts"))
 (gr_line (start 196.85 71.12) (end 199.607898 71.12) (stroke (width 0.1) (type default)) (layer "Edge.Cuts"))
 (gr_line (start 116.84 133.567898) (end 116.84 94.615) (stroke (width 0.1) (type default)) (layer "Edge.Cuts"))
 (gr_arc (start 116.84 73.66) (mid 117.583949 71.863949) (end 119.38 71.12) (stroke (width 0.05) (type default)) (layer "Edge.Cuts"))
 (gr_arc (start 200.66 73.66) (mid 199.88133 72.494638) (end 199.607898 71.12) (stroke (width 0.1) (type default)) (layer "Edge.Cuts"))
 (gr_arc (start 203.2 74.712102) (mid 201.825362 74.43867) (end 200.66 73.66) (stroke (width 0.1) (type default)) (layer "Edge.Cuts"))
 (gr_arc (start 199.644 137.16) (mid 200.685528 134.645528) (end 203.2 133.604) (stroke (width 0.1) (type default)) (layer "Edge.Cuts"))
 (gr_line (start 196.85 71.12) (end 161.29 71.12) (stroke (width 0.1) (type default)) (layer "Edge.Cuts"))
 (gr_line (start 203.2 74.712102) (end 203.2 78.74) (stroke (width 0.1) (type default)) (layer "Edge.Cuts"))
 (gr_arc (start 116.84 133.567898) (mid 118.214638 133.84133) (end 119.38 134.62) (stroke (width 0.1) (type default)) (layer "Edge.Cuts"))
 (gr_arc (start 157.48 74.93) (mid 154.785923 73.814077) (end 153.67 71.12) (stroke (width 0.05) (type default)) (layer "Edge.Cuts"))
 (segment (start 200.66 78.235) (end 200.66 76.2) (width 0.2) (layer "F.Cu") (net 7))
 (segment (start 180.34 76.965) (end 180.34 74.93) (width 0.2) (layer "F.Cu") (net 7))
 (segment (start 180.34 74.93) (end 160.02 74.93) (width 0.25) (layer "B.Cu") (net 7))
 (segment (start 180.34 76.965) (end 180.34 74.93) (width 0.2) (layer "B.Cu") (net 7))
 (segment (start 159.385 75.565) (end 159.385 85.768833) (width 0.25) (layer "B.Cu") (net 7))
 (segment (start 199.39 74.93) (end 200.66 76.2) (width 0.25) (layer "B.Cu") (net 7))
 (segment (start 200.66 78.235) (end 200.66 76.2) (width 0.2) (layer "B.Cu") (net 7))
 (segment (start 159.385 85.768833) (end 154.764433 90.3894) (width 0.25) (layer "B.Cu") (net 7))
 (segment (start 140.787 90.3894) (end 139.7 91.4764) (width 0.25) (layer "B.Cu") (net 7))
 (segment (start 154.764433 90.3894) (end 140.787 90.3894) (width 0.25) (layer "B.Cu") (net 7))
 (segment (start 180.34 74.93) (end 199.39 74.93) (width 0.25) (layer "B.Cu") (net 7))
 (segment (start 160.02 74.93) (end 159.385 75.565) (width 0.25) (layer "B.Cu") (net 7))
 (segment (start 178.565 78.74) (end 180.34 80.515) (width 0.25) (layer "F.Cu") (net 8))
 (segment (start 180.34 80.515) (end 180.34 82.55) (width 0.25) (layer "F.Cu") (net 8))
 (segment (start 172.72 78.74) (end 178.565 78.74) (width 0.25) (layer "F.Cu") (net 8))
 (segment (start 180.34 80.515) (end 180.34 82.55) (width 0.2) (layer "B.Cu") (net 8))
 (segment (start 198.25 78.74) (end 200.66 81.15) (width 0.25) (layer "F.Cu") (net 6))
 (segment (start 200.66 81.15) (end 200.66 83.185) (width 0.25) (layer "F.Cu") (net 6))
 (segment (start 193.04 78.74) (end 198.25 78.74) (width 0.25) (layer "F.Cu") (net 6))
 (segment (start 200.66 81.785) (end 200.66 83.82) (width 0.2) (layer "B.Cu") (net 6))
 (segment (start 200.66 95.25) (end 200.66 97.285) (width 0.25) (layer "F.Cu") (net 9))
 (segment (start 139.7 95.25) (end 139.7 97.285) (width 0.25) (layer "F.Cu") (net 9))
 (segment (start 160.02 95.25) (end 160.02 97.285) (width 0.25) (layer "F.Cu") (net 9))
 (segment (start 180.34 95.25) (end 180.34 97.285) (width 0.25) (layer "F.Cu") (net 9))
 (segment (start 160.02 95.25) (end 139.7 95.25) (width 0.2) (layer "B.Cu") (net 9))
 (segment (start 200.66 97.285) (end 200.66 95.25) (width 0.2) (layer "B.Cu") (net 9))
 (segment (start 180.34 97.285) (end 180.34 95.25) (width 0.2) (layer "B.Cu") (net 9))
 (segment (start 139.7 92.978295) (end 141.201895 91.4764) (width 0.2) (layer "B.Cu") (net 9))
 (segment (start 139.7 97.285) (end 139.7 95.25) (width 0.2) (layer "B.Cu") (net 9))
 (segment (start 141.201895 91.4764) (end 142.24 91.4764) (width 0.2) (layer "B.Cu") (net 9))
 (segment (start 180.34 95.25) (end 200.66 95.25) (width 0.25) (layer "B.Cu") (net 9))
 (segment (start 160.02 97.285) (end 160.02 95.25) (width 0.2) (layer "B.Cu") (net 9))
 (segment (start 139.7 95.25) (end 139.7 92.978295) (width 0.2) (layer "B.Cu") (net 9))
 (segment (start 160.02 95.25) (end 180.34 95.25) (width 0.25) (layer "B.Cu") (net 9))
 (segment (start 132.08 99.06) (end 137.925 99.06) (width 0.25) (layer "F.Cu") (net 11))
 (segment (start 137.925 99.06) (end 139.7 100.835) (width 0.25) (layer "F.Cu") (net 11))
 (segment (start 139.7 100.835) (end 139.7 102.87) (width 0.25) (layer "F.Cu") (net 11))
 (segment (start 139.7 100.835) (end 139.7 102.87) (width 0.2) (layer "B.Cu") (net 11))
 (segment (start 152.4 99.06) (end 158.245 99.06) (width 0.25) (layer "F.Cu") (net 17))
 (segment (start 158.245 99.06) (end 160.02 100.835) (width 0.25) (layer "F.Cu") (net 17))
 (segment (start 160.02 100.835) (end 160.02 102.87) (width 0.25) (layer "F.Cu") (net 17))
 (segment (start 160.02 100.835) (end 160.02 102.87) (width 0.2) (layer "B.Cu") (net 17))
 (segment (start 180.34 100.835) (end 180.34 102.87) (width 0.25) (layer "F.Cu") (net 10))
 (segment (start 178.565 99.06) (end 180.34 100.835) (width 0.25) (layer "F.Cu") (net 10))
 (segment (start 172.72 99.06) (end 178.565 99.06) (width 0.25) (layer "F.Cu") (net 10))
 (segment (start 180.34 100.835) (end 180.34 102.87) (width 0.2) (layer "B.Cu") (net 10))
 (segment (start 198.885 99.06) (end 200.66 100.835) (width 0.25) (layer "F.Cu") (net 15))
 (segment (start 193.04 99.06) (end 198.885 99.06) (width 0.25) (layer "F.Cu") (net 15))
 (segment (start 200.66 100.835) (end 200.66 102.87) (width 0.25) (layer "F.Cu") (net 15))
 (segment (start 200.66 100.835) (end 200.66 102.87) (width 0.2) (layer "B.Cu") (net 15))
 (segment (start 139.7 117.605) (end 139.7 115.57) (width 0.25) (layer "F.Cu") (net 1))
 (segment (start 140.97 93.345) (end 141.7516 92.5634) (width 0.25) (layer "F.Cu") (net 1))
 (segment (start 143.693 92.5634) (end 144.78 91.4764) (width 0.25) (layer "F.Cu") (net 1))
 (segment (start 200.66 115.57) (end 200.66 117.605) (width 0.25) (layer "F.Cu") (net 1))
 (segment (start 141.7516 92.5634) (end 143.693 92.5634) (width 0.25) (layer "F.Cu") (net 1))
 (segment (start 160.02 115.57) (end 160.02 117.605) (width 0.25) (layer "F.Cu") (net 1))
 (segment (start 140.97 97.155) (end 140.97 93.345) (width 0.25) (layer "F.Cu") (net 1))
 (segment (start 180.34 115.57) (end 180.34 117.605) (width 0.25) (layer "F.Cu") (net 1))
 (segment (start 139.7 115.57) (end 139.7 116.84) (width 0.25) (layer "F.Cu") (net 1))
 (via (at 140.97 97.155) (size 0.6) (drill 0.3) (layers "F.Cu" "B.Cu") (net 1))
 (segment (start 139.7 115.57) (end 139.7 117.605) (width 0.25) (layer "B.Cu") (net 1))
 (segment (start 143.51 115.57) (end 160.02 115.57) (width 0.25) (layer "B.Cu") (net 1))
 (segment (start 160.02 115.57) (end 160.02 117.605) (width 0.25) (layer "B.Cu") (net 1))
 (segment (start 180.34 115.57) (end 200.66 115.57) (width 0.25) (layer "B.Cu") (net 1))
 (segment (start 139.7 115.57) (end 140.97 114.3) (width 0.25) (layer "B.Cu") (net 1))
 (segment (start 160.02 115.57) (end 180.34 115.57) (width 0.25) (layer "B.Cu") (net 1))
 (segment (start 180.34 115.57) (end 180.34 117.605) (width 0.25) (layer "B.Cu") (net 1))
 (segment (start 140.97 114.3) (end 140.97 97.155) (width 0.25) (layer "B.Cu") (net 1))
 (segment (start 139.7 115.57) (end 143.51 115.57) (width 0.25) (layer "B.Cu") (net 1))
 (segment (start 200.66 117.605) (end 200.66 115.57) (width 0.2) (layer "B.Cu") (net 1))
 (segment (start 132.08 119.38) (end 137.925 119.38) (width 0.25) (layer "F.Cu") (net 4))
 (segment (start 137.925 119.38) (end 139.7 121.155) (width 0.25) (layer "F.Cu") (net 4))
 (segment (start 139.7 123.19) (end 139.7 121.155) (width 0.25) (layer "F.Cu") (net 4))
 (segment (start 139.7 121.155) (end 139.7 123.19) (width 0.2) (layer "B.Cu") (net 4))
 (segment (start 158.245 119.38) (end 160.02 121.155) (width 0.25) (layer "F.Cu") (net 16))
 (segment (start 152.4 119.38) (end 158.245 119.38) (width 0.25) (layer "F.Cu") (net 16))
 (segment (start 160.02 123.19) (end 160.02 121.155) (width 0.25) (layer "F.Cu") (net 16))
 (segment (start 160.02 121.155) (end 160.02 123.19) (width 0.2) (layer "B.Cu") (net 16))
 (segment (start 180.34 121.155) (end 180.34 123.19) (width 0.25) (layer "F.Cu") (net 19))
 (segment (start 172.72 119.38) (end 178.565 119.38) (width 0.25) (layer "F.Cu") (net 19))
 (segment (start 178.565 119.38) (end 180.34 121.155) (width 0.25) (layer "F.Cu") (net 19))
 (segment (start 180.34 121.155) (end 180.34 123.19) (width 0.2) (layer "B.Cu") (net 19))
 (segment (start 198.885 119.38) (end 200.66 121.155) (width 0.25) (layer "F.Cu") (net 2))
 (segment (start 200.66 121.155) (end 200.66 123.19) (width 0.25) (layer "F.Cu") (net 2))
 (segment (start 193.04 119.38) (end 198.885 119.38) (width 0.25) (layer "F.Cu") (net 2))
 (segment (start 200.66 121.155) (end 200.66 123.19) (width 0.2) (layer "B.Cu") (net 2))
 (segment (start 166.37 101.6) (end 166.425 101.655) (width 0.25) (layer "F.Cu") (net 12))
 (segment (start 166.425 121.865) (end 166.37 121.92) (width 0.25) (layer "F.Cu") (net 12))
 (segment (start 166.37 101.6) (end 166.425 101.545) (width 0.25) (layer "F.Cu") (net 12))
 (segment (start 166.37 78.74) (end 164.9734 77.3434) (width 0.25) (layer "F.Cu") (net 12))
 (segment (start 164.9734 77.3434) (end 140.787 77.3434) (width 0.25) (layer "F.Cu") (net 12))
 (segment (start 166.425 101.545) (end 166.425 81.335) (width 0.25) (layer "F.Cu") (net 12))
 (segment (start 166.37 81.28) (end 166.37 78.74) (width 0.25) (layer "F.Cu") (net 12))
 (segment (start 166.425 81.335) (end 166.37 81.28) (width 0.25) (layer "F.Cu") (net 12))
 (segment (start 140.787 77.3434) (end 139.7 76.2564) (width 0.25) (layer "F.Cu") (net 12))
 (segment (start 166.425 101.655) (end 166.425 121.865) (width 0.25) (layer "F.Cu") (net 12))
 (segment (start 186.69 81.28) (end 183.057448 81.28) (width 0.25) (layer "F.Cu") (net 5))
 (segment (start 186.69 81.28) (end 186.745 81.335) (width 0.25) (layer "F.Cu") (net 5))
 (segment (start 186.745 121.865) (end 186.745 101.655) (width 0.25) (layer "F.Cu") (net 5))
 (segment (start 186.745 101.655) (end 186.69 101.6) (width 0.25) (layer "F.Cu") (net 5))
 (segment (start 178.670848 76.8934) (end 154.574251 76.8934) (width 0.25) (layer "F.Cu") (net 5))
 (segment (start 183.057448 81.28) (end 178.670848 76.8934) (width 0.25) (layer "F.Cu") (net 5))
 (segment (start 154.574251 76.8934) (end 152.850251 75.1694) (width 0.25) (layer "F.Cu") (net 5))
 (segment (start 186.745 81.335) (end 186.745 101.545) (width 0.25) (layer "F.Cu") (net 5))
 (segment (start 186.745 101.545) (end 186.69 101.6) (width 0.25) (layer "F.Cu") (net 5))
 (segment (start 143.327 75.1694) (end 142.24 76.2564) (width 0.25) (layer "F.Cu") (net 5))
 (segment (start 186.69 121.92) (end 186.745 121.865) (width 0.25) (layer "F.Cu") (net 5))
 (segment (start 152.850251 75.1694) (end 143.327 75.1694) (width 0.25) (layer "F.Cu") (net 5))
 (segment (start 125.73 101.6) (end 125.785 101.655) (width 0.25) (layer "F.Cu") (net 3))
 (segment (start 126.5276 75.1944) (end 125.73 75.992) (width 0.2) (layer "F.Cu") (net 3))
 (segment (start 125.785 121.865) (end 125.73 121.92) (width 0.25) (layer "F.Cu") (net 3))
 (segment (start 125.785 101.655) (end 125.785 121.865) (width 0.25) (layer "F.Cu") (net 3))
 (segment (start 133.558 75.1944) (end 126.5276 75.1944) (width 0.2) (layer "F.Cu") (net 3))
 (segment (start 134.62 76.2564) (end 133.558 75.1944) (width 0.2) (layer "F.Cu") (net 3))
 (segment (start 125.73 75.992) (end 125.73 101.6) (width 0.2) (layer "F.Cu") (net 3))
 (segment (start 146.105 101.655) (end 146.05 101.6) (width 0.25) (layer "F.Cu") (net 18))
 (segment (start 126.18 89.119149) (end 128.087 91.026149) (width 0.25) (layer "F.Cu") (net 18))
 (segment (start 135.9464 77.47) (end 127 77.47) (width 0.25) (layer "F.Cu") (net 18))
 (segment (start 127 77.47) (end 126.18 78.29) (width 0.25) (layer "F.Cu") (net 18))
 (segment (start 126.18 78.29) (end 126.18 89.119149) (width 0.25) (layer "F.Cu") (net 18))
 (segment (start 146.05 121.92) (end 146.105 121.865) (width 0.25) (layer "F.Cu") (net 18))
 (segment (start 143.06 98.61) (end 146.05 101.6) (width 0.25) (layer "F.Cu") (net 18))
 (segment (start 137.16 76.2564) (end 135.9464 77.47) (width 0.25) (layer "F.Cu") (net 18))
 (segment (start 134.805 98.61) (end 143.06 98.61) (width 0.25) (layer "F.Cu") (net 18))
 (segment (start 128.087 91.892) (end 134.805 98.61) (width 0.25) (layer "F.Cu") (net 18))
 (segment (start 146.105 121.865) (end 146.105 101.655) (width 0.25) (layer "F.Cu") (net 18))
 (segment (start 128.087 91.026149) (end 128.087 91.892) (width 0.25) (layer "F.Cu") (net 18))
 (segment (start 156.21 87.07) (end 152.8656 90.4144) (width 0.2) (layer "F.Cu") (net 14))
 (segment (start 152.8656 90.4144) (end 133.142 90.4144) (width 0.2) (layer "F.Cu") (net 14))
 (segment (start 133.142 90.4144) (end 132.08 91.4764) (width 0.2) (layer "F.Cu") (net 14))
 (segment (start 129.54 91.4764) (end 128.2336 90.17) (width 0.25) (layer "B.Cu") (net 14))
 (segment (start 129.54 91.4764) (end 132.08 91.4764) (width 0.25) (layer "B.Cu") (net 14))
 (segment (start 125.73 77.5264) (end 127 76.2564) (width 0.25) (layer "B.Cu") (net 14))
 (segment (start 125.73 89.535) (end 125.73 77.5264) (width 0.25) (layer "B.Cu") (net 14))
 (segment (start 128.2336 90.17) (end 126.365 90.17) (width 0.25) (layer "B.Cu") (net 14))
 (segment (start 126.365 90.17) (end 125.73 89.535) (width 0.25) (layer "B.Cu") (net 14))
 (segment (start 133.167 75.1694) (end 132.08 76.2564) (width 0.25) (layer "B.Cu") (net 31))
 (segment (start 152.4 76.2564) (end 151.313 75.1694) (width 0.25) (layer "B.Cu") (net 31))
 (segment (start 151.313 75.1694) (end 133.167 75.1694) (width 0.25) (layer "B.Cu") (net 31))
 (segment (start 130.7536 77.47) (end 153.11 77.47) (width 0.25) (layer "B.Cu") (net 13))
 (segment (start 153.11 77.47) (end 156.21 80.57) (width 0.25) (layer "B.Cu") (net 13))
 (segment (start 129.54 76.2564) (end 130.7536 77.47) (width 0.25) (layer "B.Cu") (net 13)))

